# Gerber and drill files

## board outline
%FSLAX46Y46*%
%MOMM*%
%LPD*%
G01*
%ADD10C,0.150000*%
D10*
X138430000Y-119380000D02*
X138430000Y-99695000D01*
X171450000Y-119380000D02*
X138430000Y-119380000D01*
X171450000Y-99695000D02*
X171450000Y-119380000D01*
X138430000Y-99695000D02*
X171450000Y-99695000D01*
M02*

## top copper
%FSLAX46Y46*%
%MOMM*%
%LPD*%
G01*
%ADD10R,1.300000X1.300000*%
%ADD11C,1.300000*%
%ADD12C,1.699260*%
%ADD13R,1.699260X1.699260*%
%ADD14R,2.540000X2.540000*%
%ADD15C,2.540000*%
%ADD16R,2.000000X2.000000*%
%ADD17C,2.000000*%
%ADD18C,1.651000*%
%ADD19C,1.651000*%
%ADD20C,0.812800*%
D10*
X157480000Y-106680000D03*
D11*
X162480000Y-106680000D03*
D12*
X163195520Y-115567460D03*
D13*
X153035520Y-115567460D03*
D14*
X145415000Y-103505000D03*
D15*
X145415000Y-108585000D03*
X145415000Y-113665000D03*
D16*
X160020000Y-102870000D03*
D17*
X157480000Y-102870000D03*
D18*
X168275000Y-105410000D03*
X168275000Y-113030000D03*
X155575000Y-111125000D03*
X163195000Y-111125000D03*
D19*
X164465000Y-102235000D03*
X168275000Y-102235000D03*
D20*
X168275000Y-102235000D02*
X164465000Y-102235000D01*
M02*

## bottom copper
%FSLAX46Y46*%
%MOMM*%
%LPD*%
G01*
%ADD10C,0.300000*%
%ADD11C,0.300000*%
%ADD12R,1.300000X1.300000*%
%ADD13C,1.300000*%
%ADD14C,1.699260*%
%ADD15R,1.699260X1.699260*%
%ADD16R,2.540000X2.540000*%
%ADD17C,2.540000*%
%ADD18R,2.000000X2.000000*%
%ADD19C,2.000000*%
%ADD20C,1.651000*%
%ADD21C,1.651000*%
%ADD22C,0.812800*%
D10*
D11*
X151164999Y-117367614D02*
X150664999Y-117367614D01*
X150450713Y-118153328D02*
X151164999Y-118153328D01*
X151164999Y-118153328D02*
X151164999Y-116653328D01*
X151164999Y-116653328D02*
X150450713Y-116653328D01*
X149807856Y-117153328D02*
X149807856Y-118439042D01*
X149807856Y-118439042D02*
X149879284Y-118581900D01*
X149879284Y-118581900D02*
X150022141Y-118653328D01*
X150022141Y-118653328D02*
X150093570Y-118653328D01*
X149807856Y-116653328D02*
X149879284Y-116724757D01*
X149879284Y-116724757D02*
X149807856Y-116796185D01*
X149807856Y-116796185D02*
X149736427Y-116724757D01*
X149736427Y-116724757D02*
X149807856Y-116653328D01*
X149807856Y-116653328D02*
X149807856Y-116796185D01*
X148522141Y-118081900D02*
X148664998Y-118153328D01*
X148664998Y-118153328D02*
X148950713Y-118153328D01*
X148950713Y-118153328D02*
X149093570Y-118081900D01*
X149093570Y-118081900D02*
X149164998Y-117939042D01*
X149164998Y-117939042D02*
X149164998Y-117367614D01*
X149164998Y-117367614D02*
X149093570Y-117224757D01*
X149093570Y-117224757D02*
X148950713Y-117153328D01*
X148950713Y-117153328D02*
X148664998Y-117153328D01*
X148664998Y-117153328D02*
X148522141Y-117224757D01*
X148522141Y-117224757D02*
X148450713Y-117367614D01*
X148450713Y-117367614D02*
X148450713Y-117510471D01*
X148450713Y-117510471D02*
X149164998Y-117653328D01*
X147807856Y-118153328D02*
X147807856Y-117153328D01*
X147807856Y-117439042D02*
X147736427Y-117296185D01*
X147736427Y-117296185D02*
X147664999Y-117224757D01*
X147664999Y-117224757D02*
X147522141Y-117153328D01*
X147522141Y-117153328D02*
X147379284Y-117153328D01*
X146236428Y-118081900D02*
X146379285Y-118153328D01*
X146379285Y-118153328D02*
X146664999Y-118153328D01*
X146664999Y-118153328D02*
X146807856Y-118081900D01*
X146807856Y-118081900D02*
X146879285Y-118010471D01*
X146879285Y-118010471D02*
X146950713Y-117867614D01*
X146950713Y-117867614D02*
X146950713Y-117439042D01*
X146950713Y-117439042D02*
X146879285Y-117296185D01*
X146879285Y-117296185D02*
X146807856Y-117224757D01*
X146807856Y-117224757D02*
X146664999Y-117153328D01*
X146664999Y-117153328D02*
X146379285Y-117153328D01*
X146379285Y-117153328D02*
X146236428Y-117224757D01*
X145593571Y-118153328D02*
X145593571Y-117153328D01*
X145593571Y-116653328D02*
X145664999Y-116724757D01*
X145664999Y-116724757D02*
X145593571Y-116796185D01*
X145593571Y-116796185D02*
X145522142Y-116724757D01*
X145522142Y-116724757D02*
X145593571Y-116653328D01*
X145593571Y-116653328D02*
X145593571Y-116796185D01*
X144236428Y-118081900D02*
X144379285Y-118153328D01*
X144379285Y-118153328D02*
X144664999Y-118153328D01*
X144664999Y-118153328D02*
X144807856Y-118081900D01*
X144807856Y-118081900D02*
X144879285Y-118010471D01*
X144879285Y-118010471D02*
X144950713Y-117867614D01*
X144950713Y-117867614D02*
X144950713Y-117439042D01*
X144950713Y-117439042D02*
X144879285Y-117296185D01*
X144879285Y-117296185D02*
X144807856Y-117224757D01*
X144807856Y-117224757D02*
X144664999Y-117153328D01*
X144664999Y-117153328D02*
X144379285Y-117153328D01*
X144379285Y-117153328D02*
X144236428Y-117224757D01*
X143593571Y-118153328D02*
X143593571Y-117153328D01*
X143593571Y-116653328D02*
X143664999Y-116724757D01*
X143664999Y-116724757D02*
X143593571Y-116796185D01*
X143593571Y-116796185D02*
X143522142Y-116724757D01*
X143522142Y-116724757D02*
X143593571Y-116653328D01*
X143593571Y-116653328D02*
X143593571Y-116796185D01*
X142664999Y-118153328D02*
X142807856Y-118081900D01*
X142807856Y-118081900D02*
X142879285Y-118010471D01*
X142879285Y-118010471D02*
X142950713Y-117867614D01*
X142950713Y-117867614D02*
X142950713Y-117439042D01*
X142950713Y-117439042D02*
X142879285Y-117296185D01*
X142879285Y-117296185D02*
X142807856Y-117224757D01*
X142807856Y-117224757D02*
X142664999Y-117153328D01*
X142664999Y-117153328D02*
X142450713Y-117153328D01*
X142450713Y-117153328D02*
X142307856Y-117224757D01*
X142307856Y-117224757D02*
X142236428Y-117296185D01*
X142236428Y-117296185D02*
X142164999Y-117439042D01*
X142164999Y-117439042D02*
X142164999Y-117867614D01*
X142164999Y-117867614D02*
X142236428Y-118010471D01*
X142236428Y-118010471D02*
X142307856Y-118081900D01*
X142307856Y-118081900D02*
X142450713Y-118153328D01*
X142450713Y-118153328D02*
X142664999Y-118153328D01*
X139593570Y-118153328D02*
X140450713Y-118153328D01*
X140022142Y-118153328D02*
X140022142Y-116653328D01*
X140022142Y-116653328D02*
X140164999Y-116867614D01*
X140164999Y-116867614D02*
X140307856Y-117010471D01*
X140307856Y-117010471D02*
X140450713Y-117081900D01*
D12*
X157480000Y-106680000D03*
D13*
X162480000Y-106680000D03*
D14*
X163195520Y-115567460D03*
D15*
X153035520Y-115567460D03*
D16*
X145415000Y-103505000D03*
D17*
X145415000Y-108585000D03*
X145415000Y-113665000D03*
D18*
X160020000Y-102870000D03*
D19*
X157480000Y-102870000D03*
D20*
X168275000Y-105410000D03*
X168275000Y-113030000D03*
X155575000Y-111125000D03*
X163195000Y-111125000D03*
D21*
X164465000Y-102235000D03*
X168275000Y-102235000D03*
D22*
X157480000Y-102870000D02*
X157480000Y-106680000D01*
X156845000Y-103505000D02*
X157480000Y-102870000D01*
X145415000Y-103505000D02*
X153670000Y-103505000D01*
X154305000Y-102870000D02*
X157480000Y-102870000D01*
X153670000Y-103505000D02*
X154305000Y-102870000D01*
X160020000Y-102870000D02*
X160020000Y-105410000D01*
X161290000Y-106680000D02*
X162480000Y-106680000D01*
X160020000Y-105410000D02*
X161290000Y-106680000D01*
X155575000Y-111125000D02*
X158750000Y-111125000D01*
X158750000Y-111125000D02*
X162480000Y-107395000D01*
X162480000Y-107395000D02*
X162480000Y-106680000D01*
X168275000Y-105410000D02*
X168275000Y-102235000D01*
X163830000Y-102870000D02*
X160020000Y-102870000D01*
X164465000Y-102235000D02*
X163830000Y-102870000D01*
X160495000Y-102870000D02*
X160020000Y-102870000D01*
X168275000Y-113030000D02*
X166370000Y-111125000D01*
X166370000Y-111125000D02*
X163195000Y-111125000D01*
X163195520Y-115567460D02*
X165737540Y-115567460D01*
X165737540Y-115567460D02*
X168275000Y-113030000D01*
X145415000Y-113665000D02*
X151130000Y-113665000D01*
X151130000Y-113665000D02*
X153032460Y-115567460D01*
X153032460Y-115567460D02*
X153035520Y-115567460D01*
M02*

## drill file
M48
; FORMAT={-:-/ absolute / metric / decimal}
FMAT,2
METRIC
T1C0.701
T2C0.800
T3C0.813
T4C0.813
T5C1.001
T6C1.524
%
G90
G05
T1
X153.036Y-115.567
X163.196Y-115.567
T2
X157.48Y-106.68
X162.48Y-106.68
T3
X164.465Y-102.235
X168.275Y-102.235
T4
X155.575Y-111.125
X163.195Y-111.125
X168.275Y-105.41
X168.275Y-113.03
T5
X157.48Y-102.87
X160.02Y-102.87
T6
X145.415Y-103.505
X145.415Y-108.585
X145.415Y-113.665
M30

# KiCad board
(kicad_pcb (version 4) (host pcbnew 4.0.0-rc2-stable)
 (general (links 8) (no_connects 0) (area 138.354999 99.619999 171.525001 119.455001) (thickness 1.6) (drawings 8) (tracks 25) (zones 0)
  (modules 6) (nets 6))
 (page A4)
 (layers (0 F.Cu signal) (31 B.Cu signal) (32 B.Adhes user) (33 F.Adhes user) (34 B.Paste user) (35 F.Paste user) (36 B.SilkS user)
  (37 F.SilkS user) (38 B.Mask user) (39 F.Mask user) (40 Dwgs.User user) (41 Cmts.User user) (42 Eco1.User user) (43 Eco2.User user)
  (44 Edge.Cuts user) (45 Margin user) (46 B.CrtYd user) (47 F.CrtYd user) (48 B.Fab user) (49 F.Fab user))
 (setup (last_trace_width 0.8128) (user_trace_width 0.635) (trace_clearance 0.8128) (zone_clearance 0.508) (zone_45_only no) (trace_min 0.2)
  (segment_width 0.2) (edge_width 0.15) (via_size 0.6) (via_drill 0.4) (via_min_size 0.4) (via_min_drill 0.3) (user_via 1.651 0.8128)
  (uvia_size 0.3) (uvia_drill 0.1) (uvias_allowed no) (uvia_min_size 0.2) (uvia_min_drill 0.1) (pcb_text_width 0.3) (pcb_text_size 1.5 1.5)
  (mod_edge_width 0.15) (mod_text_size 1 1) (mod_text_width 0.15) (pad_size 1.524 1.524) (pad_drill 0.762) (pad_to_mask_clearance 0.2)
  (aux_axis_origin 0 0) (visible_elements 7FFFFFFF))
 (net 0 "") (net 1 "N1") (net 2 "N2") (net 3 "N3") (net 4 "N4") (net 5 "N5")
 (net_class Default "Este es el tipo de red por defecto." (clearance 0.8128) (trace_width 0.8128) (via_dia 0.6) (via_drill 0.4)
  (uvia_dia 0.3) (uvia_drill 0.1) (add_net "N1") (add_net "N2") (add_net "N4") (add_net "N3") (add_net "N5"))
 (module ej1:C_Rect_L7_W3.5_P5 (layer F.Cu) (at 157.48 106.68)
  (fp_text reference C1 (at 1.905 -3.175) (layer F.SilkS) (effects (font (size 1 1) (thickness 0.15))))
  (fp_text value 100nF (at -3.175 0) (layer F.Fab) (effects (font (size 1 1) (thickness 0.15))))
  (pad 1 thru_hole rect (at 0 0) (size 1.3 1.3) (drill 0.8) (layers *.Cu *.Mask F.SilkS) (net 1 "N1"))
  (pad 2 thru_hole circle (at 5 0) (size 1.3 1.3) (drill 0.8) (layers *.Cu *.Mask F.SilkS) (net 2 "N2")))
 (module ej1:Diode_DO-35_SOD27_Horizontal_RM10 (layer F.Cu) (at 153.035 115.57)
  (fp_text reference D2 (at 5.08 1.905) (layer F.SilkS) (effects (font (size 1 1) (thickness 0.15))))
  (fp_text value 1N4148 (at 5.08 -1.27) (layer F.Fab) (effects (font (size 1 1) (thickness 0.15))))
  (pad 2 thru_hole circle (at 10.16052 -0.00254 180) (size 1.69926 1.69926) (drill 0.70104) (layers *.Cu *.Mask F.SilkS) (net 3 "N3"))
  (pad 1 thru_hole rect (at 0.00052 -0.00254 180) (size 1.69926 1.69926) (drill 0.70104) (layers *.Cu *.Mask F.SilkS) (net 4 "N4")))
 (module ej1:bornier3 (layer F.Cu) (at 145.415 108.585 270)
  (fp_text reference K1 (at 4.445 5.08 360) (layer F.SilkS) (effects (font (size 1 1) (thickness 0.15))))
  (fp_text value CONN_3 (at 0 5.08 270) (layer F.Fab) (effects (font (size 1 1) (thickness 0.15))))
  (pad 1 thru_hole rect (at -5.08 0 270) (size 2.54 2.54) (drill 1.524) (layers *.Cu *.Mask F.SilkS) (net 1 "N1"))
  (pad 2 thru_hole circle (at 0 0 270) (size 2.54 2.54) (drill 1.524) (layers *.Cu *.Mask F.SilkS) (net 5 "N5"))
  (pad 3 thru_hole circle (at 5.08 0 270) (size 2.54 2.54) (drill 1.524) (layers *.Cu *.Mask F.SilkS) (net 4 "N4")))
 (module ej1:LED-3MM (layer F.Cu) (at 160.02 102.87 180)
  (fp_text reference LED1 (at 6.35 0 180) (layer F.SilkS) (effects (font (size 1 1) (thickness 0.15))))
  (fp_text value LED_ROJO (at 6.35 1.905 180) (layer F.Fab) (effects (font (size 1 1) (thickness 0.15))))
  (pad 1 thru_hole rect (at 0 0 270) (size 2 2) (drill 1.00076) (layers *.Cu *.Mask F.SilkS) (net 2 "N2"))
  (pad 2 thru_hole circle (at 2.54 0 180) (size 2 2) (drill 1.00076) (layers *.Cu *.Mask F.SilkS) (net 1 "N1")))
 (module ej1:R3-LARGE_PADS (layer F.Cu) (at 168.275 109.22 270)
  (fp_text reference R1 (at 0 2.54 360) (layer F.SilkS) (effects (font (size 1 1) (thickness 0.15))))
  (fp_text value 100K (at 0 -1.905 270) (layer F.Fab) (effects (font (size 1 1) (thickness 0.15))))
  (pad 1 thru_hole circle (at -3.81 0 270) (size 1.651 1.651) (drill 0.8128) (layers *.Cu *.Mask F.SilkS) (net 2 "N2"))
  (pad 2 thru_hole circle (at 3.81 0 270) (size 1.651 1.651) (drill 0.8128) (layers *.Cu *.Mask F.SilkS) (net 3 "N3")))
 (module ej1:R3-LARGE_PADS (layer F.Cu) (at 159.385 111.125)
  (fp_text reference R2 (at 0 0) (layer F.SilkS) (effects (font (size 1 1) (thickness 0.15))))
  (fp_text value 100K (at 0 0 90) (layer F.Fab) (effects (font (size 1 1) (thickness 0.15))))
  (pad 1 thru_hole circle (at -3.81 0) (size 1.651 1.651) (drill 0.8128) (layers *.Cu *.Mask F.SilkS) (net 2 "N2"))
  (pad 2 thru_hole circle (at 3.81 0) (size 1.651 1.651) (drill 0.8128) (layers *.Cu *.Mask F.SilkS) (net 3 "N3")))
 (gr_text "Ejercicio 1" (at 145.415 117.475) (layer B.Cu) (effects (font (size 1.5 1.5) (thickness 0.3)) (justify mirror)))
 (gr_line (start 138.43 119.38) (end 138.43 99.695) (angle 90) (layer Edge.Cuts) (width 0.15))
 (gr_line (start 171.45 119.38) (end 138.43 119.38) (angle 90) (layer Edge.Cuts) (width 0.15))
 (gr_line (start 171.45 99.695) (end 171.45 119.38) (angle 90) (layer Edge.Cuts) (width 0.15))
 (gr_line (start 138.43 99.695) (end 171.45 99.695) (angle 90) (layer Edge.Cuts) (width 0.15))
 (segment (start 157.48 102.87) (end 157.48 106.68) (width 0.8128) (layer B.Cu) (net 1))
 (segment (start 156.845 103.505) (end 157.48 102.87) (width 0.8128) (layer B.Cu) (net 1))
 (segment (start 145.415 103.505) (end 153.67 103.505) (width 0.8128) (layer B.Cu) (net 1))
 (segment (start 154.305 102.87) (end 157.48 102.87) (width 0.8128) (layer B.Cu) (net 1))
 (segment (start 153.67 103.505) (end 154.305 102.87) (width 0.8128) (layer B.Cu) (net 1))
 (segment (start 160.02 102.87) (end 160.02 105.41) (width 0.8128) (layer B.Cu) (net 2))
 (segment (start 161.29 106.68) (end 162.48 106.68) (width 0.8128) (layer B.Cu) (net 2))
 (segment (start 160.02 105.41) (end 161.29 106.68) (width 0.8128) (layer B.Cu) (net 2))
 (segment (start 155.575 111.125) (end 158.75 111.125) (width 0.8128) (layer B.Cu) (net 2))
 (segment (start 158.75 111.125) (end 162.48 107.395) (width 0.8128) (layer B.Cu) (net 2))
 (segment (start 162.48 107.395) (end 162.48 106.68) (width 0.8128) (layer B.Cu) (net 2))
 (segment (start 168.275 105.41) (end 168.275 102.235) (width 0.8128) (layer B.Cu) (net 2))
 (segment (start 163.83 102.87) (end 160.02 102.87) (width 0.8128) (layer B.Cu) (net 2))
 (segment (start 164.465 102.235) (end 163.83 102.87) (width 0.8128) (layer B.Cu) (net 2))
 (via (at 164.465 102.235) (size 1.651) (drill 0.8128) (layers F.Cu B.Cu) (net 2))
 (segment (start 168.275 102.235) (end 164.465 102.235) (width 0.8128) (layer F.Cu) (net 2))
 (via (at 168.275 102.235) (size 1.651) (drill 0.8128) (layers F.Cu B.Cu) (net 2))
 (segment (start 160.495 102.87) (end 160.02 102.87) (width 0.8128) (layer B.Cu) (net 2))
 (segment (start 168.275 113.03) (end 166.37 111.125) (width 0.8128) (layer B.Cu) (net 3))
 (segment (start 166.37 111.125) (end 163.195 111.125) (width 0.8128) (layer B.Cu) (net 3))
 (segment (start 163.19552 115.56746) (end 165.73754 115.56746) (width 0.8128) (layer B.Cu) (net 3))
 (segment (start 165.73754 115.56746) (end 168.275 113.03) (width 0.8128) (layer B.Cu) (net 3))
 (segment (start 145.415 113.665) (end 151.13 113.665) (width 0.8128) (layer B.Cu) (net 4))
 (segment (start 151.13 113.665) (end 153.03246 115.56746) (width 0.8128) (layer B.Cu) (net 4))
 (segment (start 153.03246 115.56746) (end 153.03552 115.56746) (width 0.8128) (layer B.Cu) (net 4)))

